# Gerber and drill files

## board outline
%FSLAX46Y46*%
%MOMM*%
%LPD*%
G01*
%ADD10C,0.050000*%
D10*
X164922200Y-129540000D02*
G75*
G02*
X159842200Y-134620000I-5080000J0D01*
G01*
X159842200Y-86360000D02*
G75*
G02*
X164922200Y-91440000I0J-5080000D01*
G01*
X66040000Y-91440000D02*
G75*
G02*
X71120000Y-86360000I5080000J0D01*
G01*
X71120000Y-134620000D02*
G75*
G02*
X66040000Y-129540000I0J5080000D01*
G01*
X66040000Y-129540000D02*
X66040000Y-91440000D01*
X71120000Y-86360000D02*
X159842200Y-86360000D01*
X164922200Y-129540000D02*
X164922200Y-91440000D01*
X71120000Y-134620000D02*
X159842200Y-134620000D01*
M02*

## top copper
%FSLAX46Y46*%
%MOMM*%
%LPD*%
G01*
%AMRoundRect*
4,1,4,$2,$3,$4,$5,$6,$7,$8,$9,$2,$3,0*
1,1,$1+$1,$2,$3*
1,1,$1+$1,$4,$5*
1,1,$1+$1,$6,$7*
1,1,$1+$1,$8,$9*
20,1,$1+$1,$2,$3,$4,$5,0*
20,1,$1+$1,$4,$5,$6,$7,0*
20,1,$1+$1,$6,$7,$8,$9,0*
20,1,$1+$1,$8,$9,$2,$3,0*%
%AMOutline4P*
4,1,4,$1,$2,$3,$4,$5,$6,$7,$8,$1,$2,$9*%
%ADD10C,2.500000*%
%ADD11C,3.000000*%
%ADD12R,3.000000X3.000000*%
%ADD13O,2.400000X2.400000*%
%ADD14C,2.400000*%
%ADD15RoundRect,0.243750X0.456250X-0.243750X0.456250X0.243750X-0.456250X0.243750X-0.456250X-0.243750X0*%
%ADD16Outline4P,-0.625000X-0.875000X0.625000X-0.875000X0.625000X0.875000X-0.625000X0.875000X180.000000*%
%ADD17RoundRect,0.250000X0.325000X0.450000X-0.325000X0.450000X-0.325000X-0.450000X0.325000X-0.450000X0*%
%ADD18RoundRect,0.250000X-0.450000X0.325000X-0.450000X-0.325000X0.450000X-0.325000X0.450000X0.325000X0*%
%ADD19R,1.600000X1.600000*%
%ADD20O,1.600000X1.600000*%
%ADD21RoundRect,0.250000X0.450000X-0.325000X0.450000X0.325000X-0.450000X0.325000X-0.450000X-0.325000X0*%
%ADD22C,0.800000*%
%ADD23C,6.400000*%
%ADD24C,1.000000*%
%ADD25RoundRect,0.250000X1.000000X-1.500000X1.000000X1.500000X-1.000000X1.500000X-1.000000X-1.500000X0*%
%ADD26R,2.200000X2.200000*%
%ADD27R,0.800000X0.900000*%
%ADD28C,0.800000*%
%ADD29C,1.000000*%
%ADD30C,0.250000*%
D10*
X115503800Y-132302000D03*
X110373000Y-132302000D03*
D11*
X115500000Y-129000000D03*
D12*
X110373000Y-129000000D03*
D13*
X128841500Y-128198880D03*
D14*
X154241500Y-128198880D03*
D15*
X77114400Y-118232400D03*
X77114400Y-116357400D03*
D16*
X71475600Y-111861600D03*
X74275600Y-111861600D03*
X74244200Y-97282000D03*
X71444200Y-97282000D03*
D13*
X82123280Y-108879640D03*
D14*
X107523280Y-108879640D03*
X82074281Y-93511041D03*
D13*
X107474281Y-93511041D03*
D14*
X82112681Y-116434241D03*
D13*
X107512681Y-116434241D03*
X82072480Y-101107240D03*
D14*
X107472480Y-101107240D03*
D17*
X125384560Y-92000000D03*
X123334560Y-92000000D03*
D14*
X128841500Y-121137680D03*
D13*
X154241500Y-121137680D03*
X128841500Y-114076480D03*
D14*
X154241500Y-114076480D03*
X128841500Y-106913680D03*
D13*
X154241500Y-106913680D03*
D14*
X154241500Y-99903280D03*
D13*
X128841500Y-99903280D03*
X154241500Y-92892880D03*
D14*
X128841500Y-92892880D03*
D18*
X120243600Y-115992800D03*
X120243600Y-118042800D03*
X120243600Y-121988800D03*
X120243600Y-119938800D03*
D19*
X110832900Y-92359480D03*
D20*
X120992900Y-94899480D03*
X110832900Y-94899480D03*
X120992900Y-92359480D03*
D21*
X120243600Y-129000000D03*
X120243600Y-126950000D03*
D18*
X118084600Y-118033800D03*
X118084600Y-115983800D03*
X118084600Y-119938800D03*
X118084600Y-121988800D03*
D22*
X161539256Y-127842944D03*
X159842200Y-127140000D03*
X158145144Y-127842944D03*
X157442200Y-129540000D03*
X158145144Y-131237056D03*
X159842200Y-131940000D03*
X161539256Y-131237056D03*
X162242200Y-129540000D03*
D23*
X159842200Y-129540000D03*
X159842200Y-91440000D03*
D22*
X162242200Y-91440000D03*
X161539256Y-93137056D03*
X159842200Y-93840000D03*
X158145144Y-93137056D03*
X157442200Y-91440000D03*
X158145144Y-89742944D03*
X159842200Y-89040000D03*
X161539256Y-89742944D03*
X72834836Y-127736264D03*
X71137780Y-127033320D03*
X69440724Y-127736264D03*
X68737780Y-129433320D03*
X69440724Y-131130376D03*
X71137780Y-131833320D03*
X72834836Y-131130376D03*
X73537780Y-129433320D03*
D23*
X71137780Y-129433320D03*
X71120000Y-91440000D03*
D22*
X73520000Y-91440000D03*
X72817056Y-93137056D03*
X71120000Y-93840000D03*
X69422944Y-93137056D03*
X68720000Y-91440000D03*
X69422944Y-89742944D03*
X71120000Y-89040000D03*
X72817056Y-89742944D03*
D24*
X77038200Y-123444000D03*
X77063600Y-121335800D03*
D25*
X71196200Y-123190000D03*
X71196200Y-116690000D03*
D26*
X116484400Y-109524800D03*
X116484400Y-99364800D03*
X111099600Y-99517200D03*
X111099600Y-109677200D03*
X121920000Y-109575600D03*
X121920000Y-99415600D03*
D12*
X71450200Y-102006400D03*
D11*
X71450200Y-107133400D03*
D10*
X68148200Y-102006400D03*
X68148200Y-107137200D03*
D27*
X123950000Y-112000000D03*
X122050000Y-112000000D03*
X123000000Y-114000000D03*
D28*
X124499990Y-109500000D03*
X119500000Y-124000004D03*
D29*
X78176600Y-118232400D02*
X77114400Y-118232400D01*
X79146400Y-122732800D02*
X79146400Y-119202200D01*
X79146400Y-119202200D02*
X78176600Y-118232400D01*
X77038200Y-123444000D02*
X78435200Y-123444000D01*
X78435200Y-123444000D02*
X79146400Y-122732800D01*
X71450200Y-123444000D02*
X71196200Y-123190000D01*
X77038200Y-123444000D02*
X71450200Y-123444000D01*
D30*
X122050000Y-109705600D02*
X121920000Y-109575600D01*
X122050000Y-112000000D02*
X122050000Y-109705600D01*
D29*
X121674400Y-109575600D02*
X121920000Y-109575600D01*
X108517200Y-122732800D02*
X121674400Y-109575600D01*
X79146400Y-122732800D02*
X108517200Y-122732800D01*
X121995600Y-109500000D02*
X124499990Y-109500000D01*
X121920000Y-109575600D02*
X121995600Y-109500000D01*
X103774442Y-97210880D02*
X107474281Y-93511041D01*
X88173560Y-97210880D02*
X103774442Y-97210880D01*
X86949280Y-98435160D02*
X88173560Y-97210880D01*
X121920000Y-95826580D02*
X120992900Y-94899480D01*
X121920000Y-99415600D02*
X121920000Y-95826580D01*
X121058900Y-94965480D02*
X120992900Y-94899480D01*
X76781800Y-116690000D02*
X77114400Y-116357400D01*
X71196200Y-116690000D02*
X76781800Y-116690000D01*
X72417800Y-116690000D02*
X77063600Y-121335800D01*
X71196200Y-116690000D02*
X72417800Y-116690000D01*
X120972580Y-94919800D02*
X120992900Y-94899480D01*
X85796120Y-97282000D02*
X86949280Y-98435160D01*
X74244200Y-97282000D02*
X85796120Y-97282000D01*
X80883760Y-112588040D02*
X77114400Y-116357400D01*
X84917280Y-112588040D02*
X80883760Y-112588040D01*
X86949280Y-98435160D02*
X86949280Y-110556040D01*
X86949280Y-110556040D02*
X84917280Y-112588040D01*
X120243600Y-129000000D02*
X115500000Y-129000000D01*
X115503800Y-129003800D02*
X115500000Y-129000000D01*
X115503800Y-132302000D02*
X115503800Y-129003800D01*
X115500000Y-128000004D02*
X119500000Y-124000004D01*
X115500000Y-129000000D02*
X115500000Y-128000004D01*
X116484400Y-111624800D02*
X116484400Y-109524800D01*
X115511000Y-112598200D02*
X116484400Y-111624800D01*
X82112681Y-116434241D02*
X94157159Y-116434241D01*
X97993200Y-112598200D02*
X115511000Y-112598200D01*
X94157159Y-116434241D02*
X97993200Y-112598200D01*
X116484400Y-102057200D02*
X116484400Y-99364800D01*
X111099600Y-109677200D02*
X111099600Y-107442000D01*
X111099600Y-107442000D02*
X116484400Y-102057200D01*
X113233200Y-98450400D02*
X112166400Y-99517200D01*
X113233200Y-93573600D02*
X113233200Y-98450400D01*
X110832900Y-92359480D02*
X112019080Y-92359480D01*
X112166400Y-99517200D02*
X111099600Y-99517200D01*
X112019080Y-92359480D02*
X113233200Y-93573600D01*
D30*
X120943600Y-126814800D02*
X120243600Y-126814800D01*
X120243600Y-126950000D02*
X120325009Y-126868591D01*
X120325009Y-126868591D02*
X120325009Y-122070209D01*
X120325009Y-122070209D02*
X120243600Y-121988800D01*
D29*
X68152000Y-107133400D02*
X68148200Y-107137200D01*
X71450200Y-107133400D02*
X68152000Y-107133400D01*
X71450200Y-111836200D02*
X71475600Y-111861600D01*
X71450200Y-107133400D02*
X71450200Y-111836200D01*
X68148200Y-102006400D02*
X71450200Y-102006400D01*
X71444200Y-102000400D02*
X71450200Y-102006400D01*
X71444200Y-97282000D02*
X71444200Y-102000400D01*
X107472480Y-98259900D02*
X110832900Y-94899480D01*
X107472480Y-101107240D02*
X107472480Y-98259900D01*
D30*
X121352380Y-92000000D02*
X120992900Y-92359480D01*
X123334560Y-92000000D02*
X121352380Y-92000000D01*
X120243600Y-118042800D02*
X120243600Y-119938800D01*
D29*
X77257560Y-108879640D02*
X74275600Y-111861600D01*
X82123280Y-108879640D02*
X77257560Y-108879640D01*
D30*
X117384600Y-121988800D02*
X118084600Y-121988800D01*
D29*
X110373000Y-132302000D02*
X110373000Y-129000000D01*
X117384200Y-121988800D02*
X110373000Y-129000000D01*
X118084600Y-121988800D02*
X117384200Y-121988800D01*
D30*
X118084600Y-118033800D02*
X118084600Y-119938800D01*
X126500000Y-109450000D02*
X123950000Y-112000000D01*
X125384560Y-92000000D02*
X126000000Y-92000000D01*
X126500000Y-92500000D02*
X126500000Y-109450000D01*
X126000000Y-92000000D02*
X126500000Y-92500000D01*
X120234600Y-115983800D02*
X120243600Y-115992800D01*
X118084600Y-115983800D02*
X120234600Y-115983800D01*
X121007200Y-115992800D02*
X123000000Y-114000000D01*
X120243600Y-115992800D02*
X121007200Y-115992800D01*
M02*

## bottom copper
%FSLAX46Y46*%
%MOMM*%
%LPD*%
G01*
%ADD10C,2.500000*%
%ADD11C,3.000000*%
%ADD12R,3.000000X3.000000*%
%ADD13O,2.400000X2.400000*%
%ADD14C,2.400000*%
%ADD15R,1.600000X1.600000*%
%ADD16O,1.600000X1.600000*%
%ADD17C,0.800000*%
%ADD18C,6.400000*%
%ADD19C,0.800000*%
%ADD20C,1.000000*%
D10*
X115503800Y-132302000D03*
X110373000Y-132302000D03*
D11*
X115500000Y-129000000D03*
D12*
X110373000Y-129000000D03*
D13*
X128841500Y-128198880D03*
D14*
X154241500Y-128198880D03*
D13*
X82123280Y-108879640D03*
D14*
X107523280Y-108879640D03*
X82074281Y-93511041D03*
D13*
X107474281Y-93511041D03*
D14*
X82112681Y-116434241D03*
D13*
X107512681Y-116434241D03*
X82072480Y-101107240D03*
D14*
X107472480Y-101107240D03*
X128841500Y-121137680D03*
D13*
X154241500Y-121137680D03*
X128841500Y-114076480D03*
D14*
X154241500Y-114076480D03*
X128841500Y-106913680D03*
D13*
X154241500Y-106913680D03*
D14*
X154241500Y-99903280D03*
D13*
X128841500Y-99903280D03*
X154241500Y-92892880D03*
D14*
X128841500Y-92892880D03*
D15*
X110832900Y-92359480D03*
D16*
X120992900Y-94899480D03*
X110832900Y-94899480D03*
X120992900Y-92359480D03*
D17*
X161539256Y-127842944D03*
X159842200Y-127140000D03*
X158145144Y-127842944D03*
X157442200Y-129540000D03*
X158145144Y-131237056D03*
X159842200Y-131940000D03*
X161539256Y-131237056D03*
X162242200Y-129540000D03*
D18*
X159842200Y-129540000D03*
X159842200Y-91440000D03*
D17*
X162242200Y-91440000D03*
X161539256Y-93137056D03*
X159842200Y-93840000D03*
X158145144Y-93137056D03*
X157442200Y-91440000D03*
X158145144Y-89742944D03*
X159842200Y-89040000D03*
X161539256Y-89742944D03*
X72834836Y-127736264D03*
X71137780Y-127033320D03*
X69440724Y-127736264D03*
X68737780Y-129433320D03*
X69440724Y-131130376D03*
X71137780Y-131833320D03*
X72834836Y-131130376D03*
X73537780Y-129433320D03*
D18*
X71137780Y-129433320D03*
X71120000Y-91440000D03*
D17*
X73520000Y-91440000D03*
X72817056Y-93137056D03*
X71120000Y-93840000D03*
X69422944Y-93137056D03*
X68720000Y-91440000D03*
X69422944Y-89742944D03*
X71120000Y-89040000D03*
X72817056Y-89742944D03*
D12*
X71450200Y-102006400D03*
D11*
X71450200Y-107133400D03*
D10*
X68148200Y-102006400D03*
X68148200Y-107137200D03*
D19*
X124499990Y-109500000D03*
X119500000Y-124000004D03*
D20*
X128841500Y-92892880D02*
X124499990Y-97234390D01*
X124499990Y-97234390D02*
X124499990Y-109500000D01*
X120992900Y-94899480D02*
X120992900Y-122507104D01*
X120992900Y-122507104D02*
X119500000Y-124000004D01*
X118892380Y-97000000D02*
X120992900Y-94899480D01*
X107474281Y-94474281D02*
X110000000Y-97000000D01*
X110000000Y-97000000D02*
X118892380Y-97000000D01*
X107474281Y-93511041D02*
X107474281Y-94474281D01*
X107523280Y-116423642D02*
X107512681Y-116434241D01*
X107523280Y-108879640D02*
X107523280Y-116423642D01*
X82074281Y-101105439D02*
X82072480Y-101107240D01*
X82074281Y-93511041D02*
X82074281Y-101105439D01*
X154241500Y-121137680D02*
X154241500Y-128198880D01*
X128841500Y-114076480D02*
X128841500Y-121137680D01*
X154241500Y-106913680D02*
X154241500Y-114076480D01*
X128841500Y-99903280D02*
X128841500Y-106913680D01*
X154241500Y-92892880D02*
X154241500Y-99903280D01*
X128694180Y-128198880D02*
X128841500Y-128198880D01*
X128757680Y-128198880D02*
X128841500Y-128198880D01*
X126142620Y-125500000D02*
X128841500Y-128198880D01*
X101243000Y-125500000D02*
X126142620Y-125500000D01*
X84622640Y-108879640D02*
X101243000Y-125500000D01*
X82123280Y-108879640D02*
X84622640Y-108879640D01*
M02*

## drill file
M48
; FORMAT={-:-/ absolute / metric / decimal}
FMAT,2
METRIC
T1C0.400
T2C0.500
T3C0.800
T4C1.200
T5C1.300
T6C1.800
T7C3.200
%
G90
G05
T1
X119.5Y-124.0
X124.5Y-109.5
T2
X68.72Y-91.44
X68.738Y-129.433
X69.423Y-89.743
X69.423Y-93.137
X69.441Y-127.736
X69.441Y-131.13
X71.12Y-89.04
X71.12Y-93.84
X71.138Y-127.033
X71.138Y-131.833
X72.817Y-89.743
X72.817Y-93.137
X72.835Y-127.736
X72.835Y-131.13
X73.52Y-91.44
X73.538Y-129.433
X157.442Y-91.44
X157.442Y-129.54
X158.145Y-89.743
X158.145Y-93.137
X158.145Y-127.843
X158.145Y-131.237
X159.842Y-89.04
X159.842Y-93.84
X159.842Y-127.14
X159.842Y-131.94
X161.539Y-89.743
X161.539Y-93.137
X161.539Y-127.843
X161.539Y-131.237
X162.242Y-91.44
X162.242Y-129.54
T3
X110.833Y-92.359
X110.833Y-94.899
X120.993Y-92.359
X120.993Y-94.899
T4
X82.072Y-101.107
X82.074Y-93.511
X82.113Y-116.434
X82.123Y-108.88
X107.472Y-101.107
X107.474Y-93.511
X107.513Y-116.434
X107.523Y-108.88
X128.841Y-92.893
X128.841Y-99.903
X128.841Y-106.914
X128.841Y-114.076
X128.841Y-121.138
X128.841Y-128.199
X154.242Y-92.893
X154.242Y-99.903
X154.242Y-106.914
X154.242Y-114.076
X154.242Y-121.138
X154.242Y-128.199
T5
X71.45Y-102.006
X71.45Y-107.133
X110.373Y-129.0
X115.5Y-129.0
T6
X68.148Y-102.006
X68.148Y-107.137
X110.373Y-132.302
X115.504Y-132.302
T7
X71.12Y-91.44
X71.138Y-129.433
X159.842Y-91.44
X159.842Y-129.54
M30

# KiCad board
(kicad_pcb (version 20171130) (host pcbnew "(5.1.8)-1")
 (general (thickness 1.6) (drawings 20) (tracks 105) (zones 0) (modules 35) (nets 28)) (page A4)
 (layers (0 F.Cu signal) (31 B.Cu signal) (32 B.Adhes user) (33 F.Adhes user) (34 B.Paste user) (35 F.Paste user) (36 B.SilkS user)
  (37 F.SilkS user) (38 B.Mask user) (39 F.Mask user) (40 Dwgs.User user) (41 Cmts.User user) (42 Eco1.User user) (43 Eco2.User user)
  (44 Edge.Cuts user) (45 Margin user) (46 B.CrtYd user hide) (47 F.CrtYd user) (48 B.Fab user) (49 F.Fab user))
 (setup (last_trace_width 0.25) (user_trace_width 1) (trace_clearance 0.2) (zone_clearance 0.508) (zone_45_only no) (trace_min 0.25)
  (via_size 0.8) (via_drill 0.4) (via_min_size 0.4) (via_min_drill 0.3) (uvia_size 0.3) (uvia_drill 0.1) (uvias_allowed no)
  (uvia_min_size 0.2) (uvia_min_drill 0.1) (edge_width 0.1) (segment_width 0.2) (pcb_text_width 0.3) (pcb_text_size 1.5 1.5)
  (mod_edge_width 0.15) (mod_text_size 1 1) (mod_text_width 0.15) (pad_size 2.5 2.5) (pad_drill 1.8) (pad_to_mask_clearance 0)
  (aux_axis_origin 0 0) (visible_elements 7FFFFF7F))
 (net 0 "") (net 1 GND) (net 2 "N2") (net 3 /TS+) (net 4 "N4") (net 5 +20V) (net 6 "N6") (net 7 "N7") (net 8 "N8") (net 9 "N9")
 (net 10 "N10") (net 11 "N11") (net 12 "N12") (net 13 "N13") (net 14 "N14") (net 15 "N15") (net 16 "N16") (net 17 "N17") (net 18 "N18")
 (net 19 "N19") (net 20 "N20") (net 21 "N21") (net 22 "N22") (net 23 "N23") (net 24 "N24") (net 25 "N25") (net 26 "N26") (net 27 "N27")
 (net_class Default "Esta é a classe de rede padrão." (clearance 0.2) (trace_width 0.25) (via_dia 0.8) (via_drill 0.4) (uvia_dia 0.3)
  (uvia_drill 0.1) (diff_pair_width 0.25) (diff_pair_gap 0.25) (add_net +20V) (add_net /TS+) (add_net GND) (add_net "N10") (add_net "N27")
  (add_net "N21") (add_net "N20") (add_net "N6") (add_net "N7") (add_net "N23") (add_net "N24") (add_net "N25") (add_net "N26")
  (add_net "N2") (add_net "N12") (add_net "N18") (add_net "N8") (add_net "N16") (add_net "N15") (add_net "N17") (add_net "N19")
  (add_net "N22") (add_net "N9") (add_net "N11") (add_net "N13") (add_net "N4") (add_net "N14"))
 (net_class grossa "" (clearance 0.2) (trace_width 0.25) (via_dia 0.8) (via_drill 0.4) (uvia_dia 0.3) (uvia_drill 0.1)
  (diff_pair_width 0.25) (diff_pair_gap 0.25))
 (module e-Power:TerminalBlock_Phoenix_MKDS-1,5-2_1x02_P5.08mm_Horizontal (layer F.Cu) (at 110.373 129)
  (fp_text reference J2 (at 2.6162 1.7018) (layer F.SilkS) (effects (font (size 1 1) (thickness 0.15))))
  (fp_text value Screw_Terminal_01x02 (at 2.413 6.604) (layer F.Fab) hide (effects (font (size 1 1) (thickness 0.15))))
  (pad 2 thru_hole circle (at 5.1308 3.302) (size 2.5 2.5) (drill 1.8) (layers *.Cu *.Mask) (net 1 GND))
  (pad 1 thru_hole circle (at 0 3.302) (size 2.5 2.5) (drill 1.8) (layers *.Cu *.Mask) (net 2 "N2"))
  (pad 2 thru_hole circle (at 5.127 0) (size 3 3) (drill 1.3) (layers *.Cu *.Mask) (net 1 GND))
  (pad 1 thru_hole rect (at 0 0) (size 3 3) (drill 1.3) (layers *.Cu *.Mask) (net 2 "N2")))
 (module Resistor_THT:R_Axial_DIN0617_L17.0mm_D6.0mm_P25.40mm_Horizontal (layer F.Cu) (at 154.2415 128.19888 180)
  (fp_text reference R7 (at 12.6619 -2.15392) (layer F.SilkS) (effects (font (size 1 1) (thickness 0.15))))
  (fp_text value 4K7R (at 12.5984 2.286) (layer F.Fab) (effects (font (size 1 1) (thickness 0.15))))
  (pad 2 thru_hole oval (at 25.4 0 180) (size 2.4 2.4) (drill 1.2) (layers *.Cu *.Mask) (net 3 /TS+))
  (pad 1 thru_hole circle (at 0 0 180) (size 2.4 2.4) (drill 1.2) (layers *.Cu *.Mask) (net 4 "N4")))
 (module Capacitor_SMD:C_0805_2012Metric (layer F.Cu) (at 77.1144 117.2949 90)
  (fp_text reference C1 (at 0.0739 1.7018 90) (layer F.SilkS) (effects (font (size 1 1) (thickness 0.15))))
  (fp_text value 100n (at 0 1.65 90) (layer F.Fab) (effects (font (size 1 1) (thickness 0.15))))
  (pad 1 smd roundrect (at -0.9375 0 90) (size 0.975 1.4) (layers F.Cu F.Paste F.Mask) (roundrect_rratio 0.25) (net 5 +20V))
  (pad 2 smd roundrect (at 0.9375 0 90) (size 0.975 1.4) (layers F.Cu F.Paste F.Mask) (roundrect_rratio 0.25) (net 1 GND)))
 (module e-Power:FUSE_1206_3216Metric (layer F.Cu) (at 72.8756 111.8616 180)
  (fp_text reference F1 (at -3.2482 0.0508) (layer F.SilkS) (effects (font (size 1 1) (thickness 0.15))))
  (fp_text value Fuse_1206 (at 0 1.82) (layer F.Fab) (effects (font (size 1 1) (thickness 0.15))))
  (pad 2 smd trapezoid (at 1.4 0 180) (size 1.25 1.75) (layers F.Cu F.Paste F.Mask) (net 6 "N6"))
  (pad 1 smd trapezoid (at -1.4 0 180) (size 1.25 1.75) (layers F.Cu F.Paste F.Mask) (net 3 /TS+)))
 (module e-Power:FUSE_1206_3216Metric (layer F.Cu) (at 72.8442 97.282 180)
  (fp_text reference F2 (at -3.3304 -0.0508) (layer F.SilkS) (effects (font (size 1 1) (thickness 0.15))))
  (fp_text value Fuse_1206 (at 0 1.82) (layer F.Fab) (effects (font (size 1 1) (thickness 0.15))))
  (pad 1 smd trapezoid (at -1.4 0 180) (size 1.25 1.75) (layers F.Cu F.Paste F.Mask) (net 1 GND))
  (pad 2 smd trapezoid (at 1.4 0 180) (size 1.25 1.75) (layers F.Cu F.Paste F.Mask) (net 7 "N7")))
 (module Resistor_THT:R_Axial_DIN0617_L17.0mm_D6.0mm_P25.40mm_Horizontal (layer F.Cu) (at 107.52328 108.87964 180)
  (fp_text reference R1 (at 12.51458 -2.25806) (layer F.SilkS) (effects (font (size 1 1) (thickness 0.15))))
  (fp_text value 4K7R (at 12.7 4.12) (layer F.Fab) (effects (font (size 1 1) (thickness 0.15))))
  (pad 2 thru_hole oval (at 25.4 0 180) (size 2.4 2.4) (drill 1.2) (layers *.Cu *.Mask) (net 3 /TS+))
  (pad 1 thru_hole circle (at 0 0 180) (size 2.4 2.4) (drill 1.2) (layers *.Cu *.Mask) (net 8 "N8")))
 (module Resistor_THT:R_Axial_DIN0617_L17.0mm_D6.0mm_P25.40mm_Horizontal (layer F.Cu) (at 82.074281 93.511041)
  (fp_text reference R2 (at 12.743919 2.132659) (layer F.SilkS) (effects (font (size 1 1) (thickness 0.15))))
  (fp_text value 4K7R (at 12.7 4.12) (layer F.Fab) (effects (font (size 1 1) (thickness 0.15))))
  (pad 1 thru_hole circle (at 0 0) (size 2.4 2.4) (drill 1.2) (layers *.Cu *.Mask) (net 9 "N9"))
  (pad 2 thru_hole oval (at 25.4 0) (size 2.4 2.4) (drill 1.2) (layers *.Cu *.Mask) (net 1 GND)))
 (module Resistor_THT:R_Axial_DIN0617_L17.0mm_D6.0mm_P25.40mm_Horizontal (layer F.Cu) (at 82.112681 116.434241)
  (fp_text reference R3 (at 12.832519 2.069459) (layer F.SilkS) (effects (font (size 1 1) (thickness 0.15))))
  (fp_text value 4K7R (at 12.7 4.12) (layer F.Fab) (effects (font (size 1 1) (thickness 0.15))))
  (pad 1 thru_hole circle (at 0 0) (size 2.4 2.4) (drill 1.2) (layers *.Cu *.Mask) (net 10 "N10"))
  (pad 2 thru_hole oval (at 25.4 0) (size 2.4 2.4) (drill 1.2) (layers *.Cu *.Mask) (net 8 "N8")))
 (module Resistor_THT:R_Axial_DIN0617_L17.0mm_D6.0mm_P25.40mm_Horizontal (layer F.Cu) (at 107.47248 101.10724 180)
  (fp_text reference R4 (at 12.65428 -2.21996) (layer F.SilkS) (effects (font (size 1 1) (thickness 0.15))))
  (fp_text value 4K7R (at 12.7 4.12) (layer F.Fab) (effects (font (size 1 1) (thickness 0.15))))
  (pad 2 thru_hole oval (at 25.4 0 180) (size 2.4 2.4) (drill 1.2) (layers *.Cu *.Mask) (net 9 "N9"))
  (pad 1 thru_hole circle (at 0 0 180) (size 2.4 2.4) (drill 1.2) (layers *.Cu *.Mask) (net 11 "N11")))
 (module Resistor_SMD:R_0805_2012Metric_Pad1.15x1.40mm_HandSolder (layer F.Cu) (at 124.35956 92 180)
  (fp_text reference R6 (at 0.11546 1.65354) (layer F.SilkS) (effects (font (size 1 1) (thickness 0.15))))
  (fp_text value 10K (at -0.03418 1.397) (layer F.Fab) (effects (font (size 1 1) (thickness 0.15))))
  (pad 1 smd roundrect (at -1.025 0 180) (size 1.15 1.4) (layers F.Cu F.Paste F.Mask) (roundrect_rratio 0.217391) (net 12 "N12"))
  (pad 2 smd roundrect (at 1.025 0 180) (size 1.15 1.4) (layers F.Cu F.Paste F.Mask) (roundrect_rratio 0.217391) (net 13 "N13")))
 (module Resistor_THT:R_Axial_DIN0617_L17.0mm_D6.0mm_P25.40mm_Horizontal (layer F.Cu) (at 128.8415 121.13768)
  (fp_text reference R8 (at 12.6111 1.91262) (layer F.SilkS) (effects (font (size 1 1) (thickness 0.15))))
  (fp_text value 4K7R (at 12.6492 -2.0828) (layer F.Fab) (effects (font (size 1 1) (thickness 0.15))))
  (pad 1 thru_hole circle (at 0 0) (size 2.4 2.4) (drill 1.2) (layers *.Cu *.Mask) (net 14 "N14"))
  (pad 2 thru_hole oval (at 25.4 0) (size 2.4 2.4) (drill 1.2) (layers *.Cu *.Mask) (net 4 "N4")))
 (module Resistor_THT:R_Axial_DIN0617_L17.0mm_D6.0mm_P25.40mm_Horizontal (layer F.Cu) (at 154.2415 114.07648 180)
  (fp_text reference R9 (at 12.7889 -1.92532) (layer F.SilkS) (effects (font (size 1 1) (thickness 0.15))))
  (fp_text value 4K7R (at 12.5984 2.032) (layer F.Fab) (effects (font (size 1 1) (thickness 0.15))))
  (pad 2 thru_hole oval (at 25.4 0 180) (size 2.4 2.4) (drill 1.2) (layers *.Cu *.Mask) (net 14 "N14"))
  (pad 1 thru_hole circle (at 0 0 180) (size 2.4 2.4) (drill 1.2) (layers *.Cu *.Mask) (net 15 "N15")))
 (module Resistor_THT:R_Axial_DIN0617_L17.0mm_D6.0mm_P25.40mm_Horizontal (layer F.Cu) (at 128.8415 106.91368)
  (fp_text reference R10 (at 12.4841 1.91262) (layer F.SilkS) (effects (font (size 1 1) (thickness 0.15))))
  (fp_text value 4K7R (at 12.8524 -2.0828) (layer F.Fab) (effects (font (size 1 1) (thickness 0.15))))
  (pad 1 thru_hole circle (at 0 0) (size 2.4 2.4) (drill 1.2) (layers *.Cu *.Mask) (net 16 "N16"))
  (pad 2 thru_hole oval (at 25.4 0) (size 2.4 2.4) (drill 1.2) (layers *.Cu *.Mask) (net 15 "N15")))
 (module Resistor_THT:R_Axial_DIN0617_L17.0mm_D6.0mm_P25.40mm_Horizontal (layer F.Cu) (at 154.2415 99.90328 180)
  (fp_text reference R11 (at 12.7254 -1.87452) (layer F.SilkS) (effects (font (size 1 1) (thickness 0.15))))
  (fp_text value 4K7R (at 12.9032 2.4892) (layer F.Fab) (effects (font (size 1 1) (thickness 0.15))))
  (pad 1 thru_hole circle (at 0 0 180) (size 2.4 2.4) (drill 1.2) (layers *.Cu *.Mask) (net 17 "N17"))
  (pad 2 thru_hole oval (at 25.4 0 180) (size 2.4 2.4) (drill 1.2) (layers *.Cu *.Mask) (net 16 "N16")))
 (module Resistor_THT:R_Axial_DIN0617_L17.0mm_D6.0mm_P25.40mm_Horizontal (layer F.Cu) (at 128.8415 92.89288)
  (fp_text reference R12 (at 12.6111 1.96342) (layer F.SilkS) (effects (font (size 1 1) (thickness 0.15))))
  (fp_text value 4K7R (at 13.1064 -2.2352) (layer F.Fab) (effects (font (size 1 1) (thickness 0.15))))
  (pad 2 thru_hole oval (at 25.4 0) (size 2.4 2.4) (drill 1.2) (layers *.Cu *.Mask) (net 17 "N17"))
  (pad 1 thru_hole circle (at 0 0) (size 2.4 2.4) (drill 1.2) (layers *.Cu *.Mask) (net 5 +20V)))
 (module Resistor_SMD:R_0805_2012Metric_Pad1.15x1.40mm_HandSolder (layer F.Cu) (at 120.2436 117.0178 270)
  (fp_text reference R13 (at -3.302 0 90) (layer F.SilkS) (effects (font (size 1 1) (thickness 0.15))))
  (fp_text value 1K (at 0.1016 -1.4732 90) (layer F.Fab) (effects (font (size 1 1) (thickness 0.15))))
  (pad 1 smd roundrect (at -1.025 0 270) (size 1.15 1.4) (layers F.Cu F.Paste F.Mask) (roundrect_rratio 0.217391) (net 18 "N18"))
  (pad 2 smd roundrect (at 1.025 0 270) (size 1.15 1.4) (layers F.Cu F.Paste F.Mask) (roundrect_rratio 0.217391) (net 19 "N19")))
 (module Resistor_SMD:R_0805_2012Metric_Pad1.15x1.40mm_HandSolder (layer F.Cu) (at 120.2436 120.9638 270)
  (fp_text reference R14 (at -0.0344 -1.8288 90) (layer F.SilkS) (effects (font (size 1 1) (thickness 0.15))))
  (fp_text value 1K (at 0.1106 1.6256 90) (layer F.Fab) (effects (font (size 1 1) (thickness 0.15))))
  (pad 2 smd roundrect (at 1.025 0 270) (size 1.15 1.4) (layers F.Cu F.Paste F.Mask) (roundrect_rratio 0.217391) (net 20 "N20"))
  (pad 1 smd roundrect (at -1.025 0 270) (size 1.15 1.4) (layers F.Cu F.Paste F.Mask) (roundrect_rratio 0.217391) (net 19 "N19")))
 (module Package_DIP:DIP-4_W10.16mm (layer F.Cu) (at 110.8329 92.35948)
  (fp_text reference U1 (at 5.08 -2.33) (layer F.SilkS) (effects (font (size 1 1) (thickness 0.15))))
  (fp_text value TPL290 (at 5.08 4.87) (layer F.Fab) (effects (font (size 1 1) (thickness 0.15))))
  (pad 1 thru_hole rect (at 0 0) (size 1.6 1.6) (drill 0.8) (layers *.Cu *.Mask) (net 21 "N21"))
  (pad 3 thru_hole oval (at 10.16 2.54) (size 1.6 1.6) (drill 0.8) (layers *.Cu *.Mask) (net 1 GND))
  (pad 2 thru_hole oval (at 0 2.54) (size 1.6 1.6) (drill 0.8) (layers *.Cu *.Mask) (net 11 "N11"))
  (pad 4 thru_hole oval (at 10.16 0) (size 1.6 1.6) (drill 0.8) (layers *.Cu *.Mask) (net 13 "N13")))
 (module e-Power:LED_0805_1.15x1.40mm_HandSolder (layer F.Cu) (at 120.2436 127.975 90)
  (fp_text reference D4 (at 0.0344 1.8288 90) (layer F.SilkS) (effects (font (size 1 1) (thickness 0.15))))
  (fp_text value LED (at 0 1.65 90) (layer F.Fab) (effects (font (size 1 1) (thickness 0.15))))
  (pad 1 smd roundrect (at -1.025 0 90) (size 1.15 1.4) (layers F.Cu F.Paste F.Mask) (roundrect_rratio 0.217391) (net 1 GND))
  (pad 2 smd roundrect (at 1.025 0 90) (size 1.15 1.4) (layers F.Cu F.Paste F.Mask) (roundrect_rratio 0.217391) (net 20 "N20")))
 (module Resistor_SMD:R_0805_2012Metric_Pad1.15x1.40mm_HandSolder (layer F.Cu) (at 118.0846 117.0088 270)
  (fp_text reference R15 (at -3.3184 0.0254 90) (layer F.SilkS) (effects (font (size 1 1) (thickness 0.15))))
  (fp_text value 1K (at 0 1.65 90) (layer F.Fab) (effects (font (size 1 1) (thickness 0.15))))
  (pad 2 smd roundrect (at 1.025 0 270) (size 1.15 1.4) (layers F.Cu F.Paste F.Mask) (roundrect_rratio 0.217391) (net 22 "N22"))
  (pad 1 smd roundrect (at -1.025 0 270) (size 1.15 1.4) (layers F.Cu F.Paste F.Mask) (roundrect_rratio 0.217391) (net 18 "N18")))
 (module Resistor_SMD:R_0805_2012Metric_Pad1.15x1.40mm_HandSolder (layer F.Cu) (at 118.0846 120.9638 270)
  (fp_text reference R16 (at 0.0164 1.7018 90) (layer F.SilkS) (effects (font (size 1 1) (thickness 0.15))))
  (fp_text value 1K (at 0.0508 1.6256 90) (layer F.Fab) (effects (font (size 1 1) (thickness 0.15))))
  (pad 1 smd roundrect (at -1.025 0 270) (size 1.15 1.4) (layers F.Cu F.Paste F.Mask) (roundrect_rratio 0.217391) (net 22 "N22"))
  (pad 2 smd roundrect (at 1.025 0 270) (size 1.15 1.4) (layers F.Cu F.Paste F.Mask) (roundrect_rratio 0.217391) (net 2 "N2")))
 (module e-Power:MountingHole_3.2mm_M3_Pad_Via (layer F.Cu) (at 159.8422 129.54)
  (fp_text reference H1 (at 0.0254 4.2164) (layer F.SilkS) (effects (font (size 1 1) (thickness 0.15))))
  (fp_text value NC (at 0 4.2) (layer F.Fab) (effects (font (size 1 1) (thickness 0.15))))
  (pad 1 thru_hole circle (at 1.697056 -1.697056) (size 0.8 0.8) (drill 0.5) (layers *.Cu *.Mask) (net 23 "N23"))
  (pad 1 thru_hole circle (at 0 -2.4) (size 0.8 0.8) (drill 0.5) (layers *.Cu *.Mask) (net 23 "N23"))
  (pad 1 thru_hole circle (at -1.697056 -1.697056) (size 0.8 0.8) (drill 0.5) (layers *.Cu *.Mask) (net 23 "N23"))
  (pad 1 thru_hole circle (at -2.4 0) (size 0.8 0.8) (drill 0.5) (layers *.Cu *.Mask) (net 23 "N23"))
  (pad 1 thru_hole circle (at -1.697056 1.697056) (size 0.8 0.8) (drill 0.5) (layers *.Cu *.Mask) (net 23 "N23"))
  (pad 1 thru_hole circle (at 0 2.4) (size 0.8 0.8) (drill 0.5) (layers *.Cu *.Mask) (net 23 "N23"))
  (pad 1 thru_hole circle (at 1.697056 1.697056) (size 0.8 0.8) (drill 0.5) (layers *.Cu *.Mask) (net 23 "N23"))
  (pad 1 thru_hole circle (at 2.4 0) (size 0.8 0.8) (drill 0.5) (layers *.Cu *.Mask) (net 23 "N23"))
  (pad 1 thru_hole circle (at 0 0) (size 6.4 6.4) (drill 3.2) (layers *.Cu *.Mask) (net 23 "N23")))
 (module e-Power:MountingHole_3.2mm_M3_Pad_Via (layer F.Cu) (at 159.8422 91.44)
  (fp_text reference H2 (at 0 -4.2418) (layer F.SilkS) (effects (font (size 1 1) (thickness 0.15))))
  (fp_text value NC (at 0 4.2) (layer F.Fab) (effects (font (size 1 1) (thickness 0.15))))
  (pad 1 thru_hole circle (at 0 0) (size 6.4 6.4) (drill 3.2) (layers *.Cu *.Mask) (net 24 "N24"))
  (pad 1 thru_hole circle (at 2.4 0) (size 0.8 0.8) (drill 0.5) (layers *.Cu *.Mask) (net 24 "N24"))
  (pad 1 thru_hole circle (at 1.697056 1.697056) (size 0.8 0.8) (drill 0.5) (layers *.Cu *.Mask) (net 24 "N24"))
  (pad 1 thru_hole circle (at 0 2.4) (size 0.8 0.8) (drill 0.5) (layers *.Cu *.Mask) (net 24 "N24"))
  (pad 1 thru_hole circle (at -1.697056 1.697056) (size 0.8 0.8) (drill 0.5) (layers *.Cu *.Mask) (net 24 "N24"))
  (pad 1 thru_hole circle (at -2.4 0) (size 0.8 0.8) (drill 0.5) (layers *.Cu *.Mask) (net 24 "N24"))
  (pad 1 thru_hole circle (at -1.697056 -1.697056) (size 0.8 0.8) (drill 0.5) (layers *.Cu *.Mask) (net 24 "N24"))
  (pad 1 thru_hole circle (at 0 -2.4) (size 0.8 0.8) (drill 0.5) (layers *.Cu *.Mask) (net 24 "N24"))
  (pad 1 thru_hole circle (at 1.697056 -1.697056) (size 0.8 0.8) (drill 0.5) (layers *.Cu *.Mask) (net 24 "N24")))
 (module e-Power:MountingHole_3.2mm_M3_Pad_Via (layer F.Cu) (at 71.13778 129.43332)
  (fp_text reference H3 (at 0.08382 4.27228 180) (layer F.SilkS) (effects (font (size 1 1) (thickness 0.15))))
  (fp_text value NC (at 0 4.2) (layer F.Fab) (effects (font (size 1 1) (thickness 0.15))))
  (pad 1 thru_hole circle (at 1.697056 -1.697056) (size 0.8 0.8) (drill 0.5) (layers *.Cu *.Mask) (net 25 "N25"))
  (pad 1 thru_hole circle (at 0 -2.4) (size 0.8 0.8) (drill 0.5) (layers *.Cu *.Mask) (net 25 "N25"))
  (pad 1 thru_hole circle (at -1.697056 -1.697056) (size 0.8 0.8) (drill 0.5) (layers *.Cu *.Mask) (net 25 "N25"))
  (pad 1 thru_hole circle (at -2.4 0) (size 0.8 0.8) (drill 0.5) (layers *.Cu *.Mask) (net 25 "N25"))
  (pad 1 thru_hole circle (at -1.697056 1.697056) (size 0.8 0.8) (drill 0.5) (layers *.Cu *.Mask) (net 25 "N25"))
  (pad 1 thru_hole circle (at 0 2.4) (size 0.8 0.8) (drill 0.5) (layers *.Cu *.Mask) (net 25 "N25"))
  (pad 1 thru_hole circle (at 1.697056 1.697056) (size 0.8 0.8) (drill 0.5) (layers *.Cu *.Mask) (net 25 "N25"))
  (pad 1 thru_hole circle (at 2.4 0) (size 0.8 0.8) (drill 0.5) (layers *.Cu *.Mask) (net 25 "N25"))
  (pad 1 thru_hole circle (at 0 0) (size 6.4 6.4) (drill 3.2) (layers *.Cu *.Mask) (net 25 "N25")))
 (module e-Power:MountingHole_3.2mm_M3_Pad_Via (layer F.Cu) (at 71.12 91.44)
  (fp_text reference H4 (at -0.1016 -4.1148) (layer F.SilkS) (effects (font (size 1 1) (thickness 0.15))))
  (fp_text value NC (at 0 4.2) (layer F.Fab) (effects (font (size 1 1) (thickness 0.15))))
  (pad 1 thru_hole circle (at 0 0) (size 6.4 6.4) (drill 3.2) (layers *.Cu *.Mask) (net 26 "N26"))
  (pad 1 thru_hole circle (at 2.4 0) (size 0.8 0.8) (drill 0.5) (layers *.Cu *.Mask) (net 26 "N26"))
  (pad 1 thru_hole circle (at 1.697056 1.697056) (size 0.8 0.8) (drill 0.5) (layers *.Cu *.Mask) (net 26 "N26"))
  (pad 1 thru_hole circle (at 0 2.4) (size 0.8 0.8) (drill 0.5) (layers *.Cu *.Mask) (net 26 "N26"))
  (pad 1 thru_hole circle (at -1.697056 1.697056) (size 0.8 0.8) (drill 0.5) (layers *.Cu *.Mask) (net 26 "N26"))
  (pad 1 thru_hole circle (at -2.4 0) (size 0.8 0.8) (drill 0.5) (layers *.Cu *.Mask) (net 26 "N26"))
  (pad 1 thru_hole circle (at -1.697056 -1.697056) (size 0.8 0.8) (drill 0.5) (layers *.Cu *.Mask) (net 26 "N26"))
  (pad 1 thru_hole circle (at 0 -2.4) (size 0.8 0.8) (drill 0.5) (layers *.Cu *.Mask) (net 26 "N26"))
  (pad 1 thru_hole circle (at 1.697056 -1.697056) (size 0.8 0.8) (drill 0.5) (layers *.Cu *.Mask) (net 26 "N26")))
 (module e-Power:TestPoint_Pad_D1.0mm (layer F.Cu) (at 77.0382 123.444)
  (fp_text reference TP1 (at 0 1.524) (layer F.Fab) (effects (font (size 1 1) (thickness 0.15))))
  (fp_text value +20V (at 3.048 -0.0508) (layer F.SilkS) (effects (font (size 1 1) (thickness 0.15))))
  (pad 1 smd circle (at 0 0) (size 1 1) (layers F.Cu F.Mask) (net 5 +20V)))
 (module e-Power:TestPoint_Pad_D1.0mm (layer F.Cu) (at 77.0636 121.3358)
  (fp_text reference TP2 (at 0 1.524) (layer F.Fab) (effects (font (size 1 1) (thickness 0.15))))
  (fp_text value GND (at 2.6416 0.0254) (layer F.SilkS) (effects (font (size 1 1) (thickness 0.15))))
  (pad 1 smd circle (at 0 0) (size 1 1) (layers F.Cu F.Mask) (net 1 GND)))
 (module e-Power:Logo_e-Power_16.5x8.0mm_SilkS (layer F.Cu) (at 83.7184 129.5908)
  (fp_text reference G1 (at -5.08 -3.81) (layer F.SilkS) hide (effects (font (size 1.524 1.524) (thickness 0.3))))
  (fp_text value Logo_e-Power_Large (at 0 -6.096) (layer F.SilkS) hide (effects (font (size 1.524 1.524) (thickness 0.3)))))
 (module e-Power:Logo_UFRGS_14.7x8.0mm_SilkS (layer F.Cu) (at 99.3902 129.3114)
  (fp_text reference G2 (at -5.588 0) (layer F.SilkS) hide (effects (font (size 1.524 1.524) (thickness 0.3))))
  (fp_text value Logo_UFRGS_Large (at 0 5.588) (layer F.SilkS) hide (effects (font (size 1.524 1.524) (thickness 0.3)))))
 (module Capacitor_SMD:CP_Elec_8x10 (layer F.Cu) (at 71.1962 119.94 90)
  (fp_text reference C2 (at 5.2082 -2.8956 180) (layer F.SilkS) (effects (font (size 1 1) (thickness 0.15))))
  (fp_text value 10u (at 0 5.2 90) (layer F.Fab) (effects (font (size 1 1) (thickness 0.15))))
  (pad 1 smd roundrect (at -3.25 0 90) (size 3.5 2.5) (layers F.Cu F.Paste F.Mask) (roundrect_rratio 0.1) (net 5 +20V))
  (pad 2 smd roundrect (at 3.25 0 90) (size 3.5 2.5) (layers F.Cu F.Paste F.Mask) (roundrect_rratio 0.1) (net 1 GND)))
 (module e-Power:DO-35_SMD (layer F.Cu) (at 116.4844 109.5248 90)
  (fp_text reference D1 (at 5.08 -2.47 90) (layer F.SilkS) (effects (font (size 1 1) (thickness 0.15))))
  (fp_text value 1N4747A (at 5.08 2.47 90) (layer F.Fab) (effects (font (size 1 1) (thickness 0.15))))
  (pad 1 smd rect (at 0 0 90) (size 2.2 2.2) (layers F.Cu F.Mask) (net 10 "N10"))
  (pad 2 smd rect (at 10.16 0 90) (size 2.2 2.2) (layers F.Cu F.Mask) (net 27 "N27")))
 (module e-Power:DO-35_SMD (layer F.Cu) (at 111.0996 109.6772 90)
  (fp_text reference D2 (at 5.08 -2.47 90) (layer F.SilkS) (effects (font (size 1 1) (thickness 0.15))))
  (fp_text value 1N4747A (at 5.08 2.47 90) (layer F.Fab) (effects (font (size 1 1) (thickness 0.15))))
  (pad 2 smd rect (at 10.16 0 90) (size 2.2 2.2) (layers F.Cu F.Mask) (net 21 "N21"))
  (pad 1 smd rect (at 0 0 90) (size 2.2 2.2) (layers F.Cu F.Mask) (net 27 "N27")))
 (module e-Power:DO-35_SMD (layer F.Cu) (at 121.92 109.5756 90)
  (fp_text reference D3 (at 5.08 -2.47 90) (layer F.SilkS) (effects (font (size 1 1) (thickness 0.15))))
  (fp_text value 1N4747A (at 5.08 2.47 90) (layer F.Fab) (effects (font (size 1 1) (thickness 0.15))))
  (pad 1 smd rect (at 0 0 90) (size 2.2 2.2) (layers F.Cu F.Mask) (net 5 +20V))
  (pad 2 smd rect (at 10.16 0 90) (size 2.2 2.2) (layers F.Cu F.Mask) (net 1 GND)))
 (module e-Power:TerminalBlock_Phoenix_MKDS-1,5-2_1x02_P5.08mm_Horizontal (layer F.Cu) (at 71.4502 102.0064 270)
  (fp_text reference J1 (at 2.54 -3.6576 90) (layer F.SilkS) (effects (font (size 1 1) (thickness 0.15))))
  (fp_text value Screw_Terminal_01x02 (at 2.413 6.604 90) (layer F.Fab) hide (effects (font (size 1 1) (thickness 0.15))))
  (pad 1 thru_hole rect (at 0 0 270) (size 3 3) (drill 1.3) (layers *.Cu *.Mask) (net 7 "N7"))
  (pad 2 thru_hole circle (at 5.127 0 270) (size 3 3) (drill 1.3) (layers *.Cu *.Mask) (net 6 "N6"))
  (pad 1 thru_hole circle (at 0 3.302 270) (size 2.5 2.5) (drill 1.8) (layers *.Cu *.Mask) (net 7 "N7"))
  (pad 2 thru_hole circle (at 5.1308 3.302 270) (size 2.5 2.5) (drill 1.8) (layers *.Cu *.Mask) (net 6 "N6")))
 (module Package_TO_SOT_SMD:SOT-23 (layer F.Cu) (at 123 113 270)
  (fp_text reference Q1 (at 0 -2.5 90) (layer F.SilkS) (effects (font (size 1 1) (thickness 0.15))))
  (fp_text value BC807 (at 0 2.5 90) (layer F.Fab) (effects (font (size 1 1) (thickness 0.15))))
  (pad 1 smd rect (at -1 -0.95 270) (size 0.9 0.8) (layers F.Cu F.Paste F.Mask) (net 12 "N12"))
  (pad 2 smd rect (at -1 0.95 270) (size 0.9 0.8) (layers F.Cu F.Paste F.Mask) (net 5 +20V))
  (pad 3 smd rect (at 1 0 270) (size 0.9 0.8) (layers F.Cu F.Paste F.Mask) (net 18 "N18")))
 (gr_arc (start 159.8422 129.54) (end 159.8422 134.62) (angle -90) (layer Edge.Cuts) (width 0.05))
 (gr_arc (start 159.8422 91.44) (end 164.9222 91.44) (angle -90) (layer Edge.Cuts) (width 0.05))
 (gr_arc (start 71.12 91.44) (end 71.12 86.36) (angle -90) (layer Edge.Cuts) (width 0.05))
 (gr_arc (start 71.12 129.54) (end 66.04 129.54) (angle -90) (layer Edge.Cuts) (width 0.05))
 (gr_line (start 66.04 129.54) (end 66.04 91.44) (layer Edge.Cuts) (width 0.05))
 (gr_line (start 71.12 86.36) (end 159.8422 86.36) (layer Edge.Cuts) (width 0.05))
 (gr_line (start 164.9222 129.54) (end 164.9222 91.44) (layer Edge.Cuts) (width 0.05))
 (gr_line (start 71.12 134.62) (end 159.8422 134.62) (layer Edge.Cuts) (width 0.05))
 (segment (start 78.1766 118.2324) (end 77.1144 118.2324) (width 1) (layer F.Cu) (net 5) (status 20))
 (segment (start 79.1464 122.7328) (end 79.1464 119.2022) (width 1) (layer F.Cu) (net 5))
 (segment (start 79.1464 119.2022) (end 78.1766 118.2324) (width 1) (layer F.Cu) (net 5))
 (segment (start 77.0382 123.444) (end 78.4352 123.444) (width 1) (layer F.Cu) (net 5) (status 10))
 (segment (start 78.4352 123.444) (end 79.1464 122.7328) (width 1) (layer F.Cu) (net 5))
 (segment (start 71.4502 123.444) (end 71.1962 123.19) (width 1) (layer F.Cu) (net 5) (status 30))
 (segment (start 77.0382 123.444) (end 71.4502 123.444) (width 1) (layer F.Cu) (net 5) (status 30))
 (segment (start 122.05 109.7056) (end 121.92 109.5756) (width 0.25) (layer F.Cu) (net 5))
 (segment (start 122.05 112) (end 122.05 109.7056) (width 0.25) (layer F.Cu) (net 5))
 (segment (start 121.6744 109.5756) (end 121.92 109.5756) (width 1) (layer F.Cu) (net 5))
 (segment (start 108.5172 122.7328) (end 121.6744 109.5756) (width 1) (layer F.Cu) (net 5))
 (segment (start 79.1464 122.7328) (end 108.5172 122.7328) (width 1) (layer F.Cu) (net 5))
 (via (at 124.49999 109.5) (size 0.8) (drill 0.4) (layers F.Cu B.Cu) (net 5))
 (segment (start 128.8415 92.89288) (end 124.49999 97.23439) (width 1) (layer B.Cu) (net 5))
 (segment (start 124.49999 97.23439) (end 124.49999 109.5) (width 1) (layer B.Cu) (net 5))
 (segment (start 121.9956 109.5) (end 124.49999 109.5) (width 1) (layer F.Cu) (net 5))
 (segment (start 121.92 109.5756) (end 121.9956 109.5) (width 1) (layer F.Cu) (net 5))
 (segment (start 103.774442 97.21088) (end 107.474281 93.511041) (width 1) (layer F.Cu) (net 1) (status 20))
 (segment (start 88.17356 97.21088) (end 103.774442 97.21088) (width 1) (layer F.Cu) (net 1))
 (segment (start 86.94928 98.43516) (end 88.17356 97.21088) (width 1) (layer F.Cu) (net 1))
 (segment (start 121.92 95.82658) (end 120.9929 94.89948) (width 1) (layer F.Cu) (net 1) (status 20))
 (segment (start 121.92 99.4156) (end 121.92 95.82658) (width 1) (layer F.Cu) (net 1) (status 10))
 (segment (start 121.0589 94.96548) (end 120.9929 94.89948) (width 1) (layer F.Cu) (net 1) (status 30))
 (segment (start 76.7818 116.69) (end 77.1144 116.3574) (width 1) (layer F.Cu) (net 1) (status 30))
 (segment (start 71.1962 116.69) (end 76.7818 116.69) (width 1) (layer F.Cu) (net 1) (status 30))
 (segment (start 72.4178 116.69) (end 77.0636 121.3358) (width 1) (layer F.Cu) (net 1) (status 30))
 (segment (start 71.1962 116.69) (end 72.4178 116.69) (width 1) (layer F.Cu) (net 1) (status 30))
 (segment (start 120.97258 94.9198) (end 120.9929 94.89948) (width 1) (layer F.Cu) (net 1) (status 30))
 (segment (start 85.79612 97.282) (end 86.94928 98.43516) (width 1) (layer F.Cu) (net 1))
 (segment (start 74.2442 97.282) (end 85.79612 97.282) (width 1) (layer F.Cu) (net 1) (status 10))
 (segment (start 80.88376 112.58804) (end 77.1144 116.3574) (width 1) (layer F.Cu) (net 1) (status 20))
 (segment (start 84.91728 112.58804) (end 80.88376 112.58804) (width 1) (layer F.Cu) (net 1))
 (segment (start 86.94928 98.43516) (end 86.94928 110.55604) (width 1) (layer F.Cu) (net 1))
 (segment (start 86.94928 110.55604) (end 84.91728 112.58804) (width 1) (layer F.Cu) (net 1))
 (segment (start 120.2436 129) (end 115.5 129) (width 1) (layer F.Cu) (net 1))
 (segment (start 115.5038 129.0038) (end 115.5 129) (width 1) (layer F.Cu) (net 1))
 (segment (start 115.5038 132.302) (end 115.5038 129.0038) (width 1) (layer F.Cu) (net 1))
 (via (at 119.5 124.000004) (size 0.8) (drill 0.4) (layers F.Cu B.Cu) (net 1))
 (segment (start 120.9929 94.89948) (end 120.9929 122.507104) (width 1) (layer B.Cu) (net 1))
 (segment (start 120.9929 122.507104) (end 119.5 124.000004) (width 1) (layer B.Cu) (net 1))
 (segment (start 115.5 128.000004) (end 119.5 124.000004) (width 1) (layer F.Cu) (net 1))
 (segment (start 115.5 129) (end 115.5 128.000004) (width 1) (layer F.Cu) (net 1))
 (segment (start 118.89238 97) (end 120.9929 94.89948) (width 1) (layer B.Cu) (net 1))
 (segment (start 107.474281 94.474281) (end 110 97) (width 1) (layer B.Cu) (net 1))
 (segment (start 110 97) (end 118.89238 97) (width 1) (layer B.Cu) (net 1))
 (segment (start 107.474281 93.511041) (end 107.474281 94.474281) (width 1) (layer B.Cu) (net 1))
 (segment (start 116.4844 111.6248) (end 116.4844 109.5248) (width 1) (layer F.Cu) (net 10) (status 20))
 (segment (start 115.511 112.5982) (end 116.4844 111.6248) (width 1) (layer F.Cu) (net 10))
 (segment (start 82.112681 116.434241) (end 94.157159 116.434241) (width 1) (layer F.Cu) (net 10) (status 10))
 (segment (start 97.9932 112.5982) (end 115.511 112.5982) (width 1) (layer F.Cu) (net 10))
 (segment (start 94.157159 116.434241) (end 97.9932 112.5982) (width 1) (layer F.Cu) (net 10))
 (segment (start 116.4844 102.0572) (end 116.4844 99.3648) (width 1) (layer F.Cu) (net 27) (status 20))
 (segment (start 111.0996 109.6772) (end 111.0996 107.442) (width 1) (layer F.Cu) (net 27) (status 10))
 (segment (start 111.0996 107.442) (end 116.4844 102.0572) (width 1) (layer F.Cu) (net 27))
 (segment (start 113.2332 98.4504) (end 112.1664 99.5172) (width 1) (layer F.Cu) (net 21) (status 20))
 (segment (start 113.2332 93.5736) (end 113.2332 98.4504) (width 1) (layer F.Cu) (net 21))
 (segment (start 110.8329 92.35948) (end 112.01908 92.35948) (width 1) (layer F.Cu) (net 21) (status 10))
 (segment (start 112.1664 99.5172) (end 111.0996 99.5172) (width 1) (layer F.Cu) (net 21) (status 30))
 (segment (start 112.01908 92.35948) (end 113.2332 93.5736) (width 1) (layer F.Cu) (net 21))
 (segment (start 120.9436 126.8148) (end 120.2436 126.8148) (width 0.25) (layer F.Cu) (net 20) (status 20))
 (segment (start 120.2436 126.95) (end 120.325009 126.868591) (width 0.25) (layer F.Cu) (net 20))
 (segment (start 120.325009 126.868591) (end 120.325009 122.070209) (width 0.25) (layer F.Cu) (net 20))
 (segment (start 120.325009 122.070209) (end 120.2436 121.9888) (width 0.25) (layer F.Cu) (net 20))
 (segment (start 68.152 107.1334) (end 68.1482 107.1372) (width 1) (layer F.Cu) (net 6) (status 30))
 (segment (start 71.4502 107.1334) (end 68.152 107.1334) (width 1) (layer F.Cu) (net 6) (status 30))
 (segment (start 71.4502 111.8362) (end 71.4756 111.8616) (width 1) (layer F.Cu) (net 6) (status 30))
 (segment (start 71.4502 107.1334) (end 71.4502 111.8362) (width 1) (layer F.Cu) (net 6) (status 30))
 (segment (start 68.1482 102.0064) (end 71.4502 102.0064) (width 1) (layer F.Cu) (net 7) (status 30))
 (segment (start 71.4442 102.0004) (end 71.4502 102.0064) (width 1) (layer F.Cu) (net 7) (status 30))
 (segment (start 71.4442 97.282) (end 71.4442 102.0004) (width 1) (layer F.Cu) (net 7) (status 30))
 (segment (start 107.52328 116.423642) (end 107.512681 116.434241) (width 1) (layer B.Cu) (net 8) (status 30))
 (segment (start 107.52328 108.87964) (end 107.52328 116.423642) (width 1) (layer B.Cu) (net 8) (status 30))
 (segment (start 82.074281 101.105439) (end 82.07248 101.10724) (width 1) (layer B.Cu) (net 9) (status 30))
 (segment (start 82.074281 93.511041) (end 82.074281 101.105439) (width 1) (layer B.Cu) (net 9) (status 30))
 (segment (start 107.47248 98.2599) (end 110.8329 94.89948) (width 1) (layer F.Cu) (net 11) (status 20))
 (segment (start 107.47248 101.10724) (end 107.47248 98.2599) (width 1) (layer F.Cu) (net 11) (status 10))
 (segment (start 121.35238 92) (end 120.9929 92.35948) (width 0.25) (layer F.Cu) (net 13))
 (segment (start 123.33456 92) (end 121.35238 92) (width 0.25) (layer F.Cu) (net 13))
 (segment (start 154.2415 121.13768) (end 154.2415 128.19888) (width 1) (layer B.Cu) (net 4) (status 30))
 (segment (start 128.8415 114.07648) (end 128.8415 121.13768) (width 1) (layer B.Cu) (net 14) (status 30))
 (segment (start 154.2415 106.91368) (end 154.2415 114.07648) (width 1) (layer B.Cu) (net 15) (status 30))
 (segment (start 128.8415 99.90328) (end 128.8415 106.91368) (width 1) (layer B.Cu) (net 16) (status 30))
 (segment (start 154.2415 92.89288) (end 154.2415 99.90328) (width 1) (layer B.Cu) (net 17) (status 30))
 (segment (start 120.2436 118.0428) (end 120.2436 119.9388) (width 0.25) (layer F.Cu) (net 19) (status 30))
 (segment (start 128.69418 128.19888) (end 128.8415 128.19888) (width 1) (layer B.Cu) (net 3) (status 30))
 (segment (start 128.75768 128.19888) (end 128.8415 128.19888) (width 1) (layer B.Cu) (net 3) (status 30))
 (segment (start 77.25756 108.87964) (end 74.2756 111.8616) (width 1) (layer F.Cu) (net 3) (status 20))
 (segment (start 82.12328 108.87964) (end 77.25756 108.87964) (width 1) (layer F.Cu) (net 3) (status 10))
 (segment (start 126.14262 125.5) (end 128.8415 128.19888) (width 1) (layer B.Cu) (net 3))
 (segment (start 101.243 125.5) (end 126.14262 125.5) (width 1) (layer B.Cu) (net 3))
 (segment (start 84.62264 108.87964) (end 101.243 125.5) (width 1) (layer B.Cu) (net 3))
 (segment (start 82.12328 108.87964) (end 84.62264 108.87964) (width 1) (layer B.Cu) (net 3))
 (segment (start 117.3846 121.9888) (end 118.0846 121.9888) (width 0.25) (layer F.Cu) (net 2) (status 30))
 (segment (start 110.373 132.302) (end 110.373 129) (width 1) (layer F.Cu) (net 2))
 (segment (start 117.3842 121.9888) (end 110.373 129) (width 1) (layer F.Cu) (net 2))
 (segment (start 118.0846 121.9888) (end 117.3842 121.9888) (width 1) (layer F.Cu) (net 2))
 (segment (start 118.0846 118.0338) (end 118.0846 119.9388) (width 0.25) (layer F.Cu) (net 22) (status 30))
 (segment (start 126.5 109.45) (end 123.95 112) (width 0.25) (layer F.Cu) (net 12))
 (segment (start 125.38456 92) (end 126 92) (width 0.25) (layer F.Cu) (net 12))
 (segment (start 126.5 92.5) (end 126.5 109.45) (width 0.25) (layer F.Cu) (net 12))
 (segment (start 126 92) (end 126.5 92.5) (width 0.25) (layer F.Cu) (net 12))
 (segment (start 120.2346 115.9838) (end 120.2436 115.9928) (width 0.25) (layer F.Cu) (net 18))
 (segment (start 118.0846 115.9838) (end 120.2346 115.9838) (width 0.25) (layer F.Cu) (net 18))
 (segment (start 121.0072 115.9928) (end 123 114) (width 0.25) (layer F.Cu) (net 18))
 (segment (start 120.2436 115.9928) (end 121.0072 115.9928) (width 0.25) (layer F.Cu) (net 18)))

